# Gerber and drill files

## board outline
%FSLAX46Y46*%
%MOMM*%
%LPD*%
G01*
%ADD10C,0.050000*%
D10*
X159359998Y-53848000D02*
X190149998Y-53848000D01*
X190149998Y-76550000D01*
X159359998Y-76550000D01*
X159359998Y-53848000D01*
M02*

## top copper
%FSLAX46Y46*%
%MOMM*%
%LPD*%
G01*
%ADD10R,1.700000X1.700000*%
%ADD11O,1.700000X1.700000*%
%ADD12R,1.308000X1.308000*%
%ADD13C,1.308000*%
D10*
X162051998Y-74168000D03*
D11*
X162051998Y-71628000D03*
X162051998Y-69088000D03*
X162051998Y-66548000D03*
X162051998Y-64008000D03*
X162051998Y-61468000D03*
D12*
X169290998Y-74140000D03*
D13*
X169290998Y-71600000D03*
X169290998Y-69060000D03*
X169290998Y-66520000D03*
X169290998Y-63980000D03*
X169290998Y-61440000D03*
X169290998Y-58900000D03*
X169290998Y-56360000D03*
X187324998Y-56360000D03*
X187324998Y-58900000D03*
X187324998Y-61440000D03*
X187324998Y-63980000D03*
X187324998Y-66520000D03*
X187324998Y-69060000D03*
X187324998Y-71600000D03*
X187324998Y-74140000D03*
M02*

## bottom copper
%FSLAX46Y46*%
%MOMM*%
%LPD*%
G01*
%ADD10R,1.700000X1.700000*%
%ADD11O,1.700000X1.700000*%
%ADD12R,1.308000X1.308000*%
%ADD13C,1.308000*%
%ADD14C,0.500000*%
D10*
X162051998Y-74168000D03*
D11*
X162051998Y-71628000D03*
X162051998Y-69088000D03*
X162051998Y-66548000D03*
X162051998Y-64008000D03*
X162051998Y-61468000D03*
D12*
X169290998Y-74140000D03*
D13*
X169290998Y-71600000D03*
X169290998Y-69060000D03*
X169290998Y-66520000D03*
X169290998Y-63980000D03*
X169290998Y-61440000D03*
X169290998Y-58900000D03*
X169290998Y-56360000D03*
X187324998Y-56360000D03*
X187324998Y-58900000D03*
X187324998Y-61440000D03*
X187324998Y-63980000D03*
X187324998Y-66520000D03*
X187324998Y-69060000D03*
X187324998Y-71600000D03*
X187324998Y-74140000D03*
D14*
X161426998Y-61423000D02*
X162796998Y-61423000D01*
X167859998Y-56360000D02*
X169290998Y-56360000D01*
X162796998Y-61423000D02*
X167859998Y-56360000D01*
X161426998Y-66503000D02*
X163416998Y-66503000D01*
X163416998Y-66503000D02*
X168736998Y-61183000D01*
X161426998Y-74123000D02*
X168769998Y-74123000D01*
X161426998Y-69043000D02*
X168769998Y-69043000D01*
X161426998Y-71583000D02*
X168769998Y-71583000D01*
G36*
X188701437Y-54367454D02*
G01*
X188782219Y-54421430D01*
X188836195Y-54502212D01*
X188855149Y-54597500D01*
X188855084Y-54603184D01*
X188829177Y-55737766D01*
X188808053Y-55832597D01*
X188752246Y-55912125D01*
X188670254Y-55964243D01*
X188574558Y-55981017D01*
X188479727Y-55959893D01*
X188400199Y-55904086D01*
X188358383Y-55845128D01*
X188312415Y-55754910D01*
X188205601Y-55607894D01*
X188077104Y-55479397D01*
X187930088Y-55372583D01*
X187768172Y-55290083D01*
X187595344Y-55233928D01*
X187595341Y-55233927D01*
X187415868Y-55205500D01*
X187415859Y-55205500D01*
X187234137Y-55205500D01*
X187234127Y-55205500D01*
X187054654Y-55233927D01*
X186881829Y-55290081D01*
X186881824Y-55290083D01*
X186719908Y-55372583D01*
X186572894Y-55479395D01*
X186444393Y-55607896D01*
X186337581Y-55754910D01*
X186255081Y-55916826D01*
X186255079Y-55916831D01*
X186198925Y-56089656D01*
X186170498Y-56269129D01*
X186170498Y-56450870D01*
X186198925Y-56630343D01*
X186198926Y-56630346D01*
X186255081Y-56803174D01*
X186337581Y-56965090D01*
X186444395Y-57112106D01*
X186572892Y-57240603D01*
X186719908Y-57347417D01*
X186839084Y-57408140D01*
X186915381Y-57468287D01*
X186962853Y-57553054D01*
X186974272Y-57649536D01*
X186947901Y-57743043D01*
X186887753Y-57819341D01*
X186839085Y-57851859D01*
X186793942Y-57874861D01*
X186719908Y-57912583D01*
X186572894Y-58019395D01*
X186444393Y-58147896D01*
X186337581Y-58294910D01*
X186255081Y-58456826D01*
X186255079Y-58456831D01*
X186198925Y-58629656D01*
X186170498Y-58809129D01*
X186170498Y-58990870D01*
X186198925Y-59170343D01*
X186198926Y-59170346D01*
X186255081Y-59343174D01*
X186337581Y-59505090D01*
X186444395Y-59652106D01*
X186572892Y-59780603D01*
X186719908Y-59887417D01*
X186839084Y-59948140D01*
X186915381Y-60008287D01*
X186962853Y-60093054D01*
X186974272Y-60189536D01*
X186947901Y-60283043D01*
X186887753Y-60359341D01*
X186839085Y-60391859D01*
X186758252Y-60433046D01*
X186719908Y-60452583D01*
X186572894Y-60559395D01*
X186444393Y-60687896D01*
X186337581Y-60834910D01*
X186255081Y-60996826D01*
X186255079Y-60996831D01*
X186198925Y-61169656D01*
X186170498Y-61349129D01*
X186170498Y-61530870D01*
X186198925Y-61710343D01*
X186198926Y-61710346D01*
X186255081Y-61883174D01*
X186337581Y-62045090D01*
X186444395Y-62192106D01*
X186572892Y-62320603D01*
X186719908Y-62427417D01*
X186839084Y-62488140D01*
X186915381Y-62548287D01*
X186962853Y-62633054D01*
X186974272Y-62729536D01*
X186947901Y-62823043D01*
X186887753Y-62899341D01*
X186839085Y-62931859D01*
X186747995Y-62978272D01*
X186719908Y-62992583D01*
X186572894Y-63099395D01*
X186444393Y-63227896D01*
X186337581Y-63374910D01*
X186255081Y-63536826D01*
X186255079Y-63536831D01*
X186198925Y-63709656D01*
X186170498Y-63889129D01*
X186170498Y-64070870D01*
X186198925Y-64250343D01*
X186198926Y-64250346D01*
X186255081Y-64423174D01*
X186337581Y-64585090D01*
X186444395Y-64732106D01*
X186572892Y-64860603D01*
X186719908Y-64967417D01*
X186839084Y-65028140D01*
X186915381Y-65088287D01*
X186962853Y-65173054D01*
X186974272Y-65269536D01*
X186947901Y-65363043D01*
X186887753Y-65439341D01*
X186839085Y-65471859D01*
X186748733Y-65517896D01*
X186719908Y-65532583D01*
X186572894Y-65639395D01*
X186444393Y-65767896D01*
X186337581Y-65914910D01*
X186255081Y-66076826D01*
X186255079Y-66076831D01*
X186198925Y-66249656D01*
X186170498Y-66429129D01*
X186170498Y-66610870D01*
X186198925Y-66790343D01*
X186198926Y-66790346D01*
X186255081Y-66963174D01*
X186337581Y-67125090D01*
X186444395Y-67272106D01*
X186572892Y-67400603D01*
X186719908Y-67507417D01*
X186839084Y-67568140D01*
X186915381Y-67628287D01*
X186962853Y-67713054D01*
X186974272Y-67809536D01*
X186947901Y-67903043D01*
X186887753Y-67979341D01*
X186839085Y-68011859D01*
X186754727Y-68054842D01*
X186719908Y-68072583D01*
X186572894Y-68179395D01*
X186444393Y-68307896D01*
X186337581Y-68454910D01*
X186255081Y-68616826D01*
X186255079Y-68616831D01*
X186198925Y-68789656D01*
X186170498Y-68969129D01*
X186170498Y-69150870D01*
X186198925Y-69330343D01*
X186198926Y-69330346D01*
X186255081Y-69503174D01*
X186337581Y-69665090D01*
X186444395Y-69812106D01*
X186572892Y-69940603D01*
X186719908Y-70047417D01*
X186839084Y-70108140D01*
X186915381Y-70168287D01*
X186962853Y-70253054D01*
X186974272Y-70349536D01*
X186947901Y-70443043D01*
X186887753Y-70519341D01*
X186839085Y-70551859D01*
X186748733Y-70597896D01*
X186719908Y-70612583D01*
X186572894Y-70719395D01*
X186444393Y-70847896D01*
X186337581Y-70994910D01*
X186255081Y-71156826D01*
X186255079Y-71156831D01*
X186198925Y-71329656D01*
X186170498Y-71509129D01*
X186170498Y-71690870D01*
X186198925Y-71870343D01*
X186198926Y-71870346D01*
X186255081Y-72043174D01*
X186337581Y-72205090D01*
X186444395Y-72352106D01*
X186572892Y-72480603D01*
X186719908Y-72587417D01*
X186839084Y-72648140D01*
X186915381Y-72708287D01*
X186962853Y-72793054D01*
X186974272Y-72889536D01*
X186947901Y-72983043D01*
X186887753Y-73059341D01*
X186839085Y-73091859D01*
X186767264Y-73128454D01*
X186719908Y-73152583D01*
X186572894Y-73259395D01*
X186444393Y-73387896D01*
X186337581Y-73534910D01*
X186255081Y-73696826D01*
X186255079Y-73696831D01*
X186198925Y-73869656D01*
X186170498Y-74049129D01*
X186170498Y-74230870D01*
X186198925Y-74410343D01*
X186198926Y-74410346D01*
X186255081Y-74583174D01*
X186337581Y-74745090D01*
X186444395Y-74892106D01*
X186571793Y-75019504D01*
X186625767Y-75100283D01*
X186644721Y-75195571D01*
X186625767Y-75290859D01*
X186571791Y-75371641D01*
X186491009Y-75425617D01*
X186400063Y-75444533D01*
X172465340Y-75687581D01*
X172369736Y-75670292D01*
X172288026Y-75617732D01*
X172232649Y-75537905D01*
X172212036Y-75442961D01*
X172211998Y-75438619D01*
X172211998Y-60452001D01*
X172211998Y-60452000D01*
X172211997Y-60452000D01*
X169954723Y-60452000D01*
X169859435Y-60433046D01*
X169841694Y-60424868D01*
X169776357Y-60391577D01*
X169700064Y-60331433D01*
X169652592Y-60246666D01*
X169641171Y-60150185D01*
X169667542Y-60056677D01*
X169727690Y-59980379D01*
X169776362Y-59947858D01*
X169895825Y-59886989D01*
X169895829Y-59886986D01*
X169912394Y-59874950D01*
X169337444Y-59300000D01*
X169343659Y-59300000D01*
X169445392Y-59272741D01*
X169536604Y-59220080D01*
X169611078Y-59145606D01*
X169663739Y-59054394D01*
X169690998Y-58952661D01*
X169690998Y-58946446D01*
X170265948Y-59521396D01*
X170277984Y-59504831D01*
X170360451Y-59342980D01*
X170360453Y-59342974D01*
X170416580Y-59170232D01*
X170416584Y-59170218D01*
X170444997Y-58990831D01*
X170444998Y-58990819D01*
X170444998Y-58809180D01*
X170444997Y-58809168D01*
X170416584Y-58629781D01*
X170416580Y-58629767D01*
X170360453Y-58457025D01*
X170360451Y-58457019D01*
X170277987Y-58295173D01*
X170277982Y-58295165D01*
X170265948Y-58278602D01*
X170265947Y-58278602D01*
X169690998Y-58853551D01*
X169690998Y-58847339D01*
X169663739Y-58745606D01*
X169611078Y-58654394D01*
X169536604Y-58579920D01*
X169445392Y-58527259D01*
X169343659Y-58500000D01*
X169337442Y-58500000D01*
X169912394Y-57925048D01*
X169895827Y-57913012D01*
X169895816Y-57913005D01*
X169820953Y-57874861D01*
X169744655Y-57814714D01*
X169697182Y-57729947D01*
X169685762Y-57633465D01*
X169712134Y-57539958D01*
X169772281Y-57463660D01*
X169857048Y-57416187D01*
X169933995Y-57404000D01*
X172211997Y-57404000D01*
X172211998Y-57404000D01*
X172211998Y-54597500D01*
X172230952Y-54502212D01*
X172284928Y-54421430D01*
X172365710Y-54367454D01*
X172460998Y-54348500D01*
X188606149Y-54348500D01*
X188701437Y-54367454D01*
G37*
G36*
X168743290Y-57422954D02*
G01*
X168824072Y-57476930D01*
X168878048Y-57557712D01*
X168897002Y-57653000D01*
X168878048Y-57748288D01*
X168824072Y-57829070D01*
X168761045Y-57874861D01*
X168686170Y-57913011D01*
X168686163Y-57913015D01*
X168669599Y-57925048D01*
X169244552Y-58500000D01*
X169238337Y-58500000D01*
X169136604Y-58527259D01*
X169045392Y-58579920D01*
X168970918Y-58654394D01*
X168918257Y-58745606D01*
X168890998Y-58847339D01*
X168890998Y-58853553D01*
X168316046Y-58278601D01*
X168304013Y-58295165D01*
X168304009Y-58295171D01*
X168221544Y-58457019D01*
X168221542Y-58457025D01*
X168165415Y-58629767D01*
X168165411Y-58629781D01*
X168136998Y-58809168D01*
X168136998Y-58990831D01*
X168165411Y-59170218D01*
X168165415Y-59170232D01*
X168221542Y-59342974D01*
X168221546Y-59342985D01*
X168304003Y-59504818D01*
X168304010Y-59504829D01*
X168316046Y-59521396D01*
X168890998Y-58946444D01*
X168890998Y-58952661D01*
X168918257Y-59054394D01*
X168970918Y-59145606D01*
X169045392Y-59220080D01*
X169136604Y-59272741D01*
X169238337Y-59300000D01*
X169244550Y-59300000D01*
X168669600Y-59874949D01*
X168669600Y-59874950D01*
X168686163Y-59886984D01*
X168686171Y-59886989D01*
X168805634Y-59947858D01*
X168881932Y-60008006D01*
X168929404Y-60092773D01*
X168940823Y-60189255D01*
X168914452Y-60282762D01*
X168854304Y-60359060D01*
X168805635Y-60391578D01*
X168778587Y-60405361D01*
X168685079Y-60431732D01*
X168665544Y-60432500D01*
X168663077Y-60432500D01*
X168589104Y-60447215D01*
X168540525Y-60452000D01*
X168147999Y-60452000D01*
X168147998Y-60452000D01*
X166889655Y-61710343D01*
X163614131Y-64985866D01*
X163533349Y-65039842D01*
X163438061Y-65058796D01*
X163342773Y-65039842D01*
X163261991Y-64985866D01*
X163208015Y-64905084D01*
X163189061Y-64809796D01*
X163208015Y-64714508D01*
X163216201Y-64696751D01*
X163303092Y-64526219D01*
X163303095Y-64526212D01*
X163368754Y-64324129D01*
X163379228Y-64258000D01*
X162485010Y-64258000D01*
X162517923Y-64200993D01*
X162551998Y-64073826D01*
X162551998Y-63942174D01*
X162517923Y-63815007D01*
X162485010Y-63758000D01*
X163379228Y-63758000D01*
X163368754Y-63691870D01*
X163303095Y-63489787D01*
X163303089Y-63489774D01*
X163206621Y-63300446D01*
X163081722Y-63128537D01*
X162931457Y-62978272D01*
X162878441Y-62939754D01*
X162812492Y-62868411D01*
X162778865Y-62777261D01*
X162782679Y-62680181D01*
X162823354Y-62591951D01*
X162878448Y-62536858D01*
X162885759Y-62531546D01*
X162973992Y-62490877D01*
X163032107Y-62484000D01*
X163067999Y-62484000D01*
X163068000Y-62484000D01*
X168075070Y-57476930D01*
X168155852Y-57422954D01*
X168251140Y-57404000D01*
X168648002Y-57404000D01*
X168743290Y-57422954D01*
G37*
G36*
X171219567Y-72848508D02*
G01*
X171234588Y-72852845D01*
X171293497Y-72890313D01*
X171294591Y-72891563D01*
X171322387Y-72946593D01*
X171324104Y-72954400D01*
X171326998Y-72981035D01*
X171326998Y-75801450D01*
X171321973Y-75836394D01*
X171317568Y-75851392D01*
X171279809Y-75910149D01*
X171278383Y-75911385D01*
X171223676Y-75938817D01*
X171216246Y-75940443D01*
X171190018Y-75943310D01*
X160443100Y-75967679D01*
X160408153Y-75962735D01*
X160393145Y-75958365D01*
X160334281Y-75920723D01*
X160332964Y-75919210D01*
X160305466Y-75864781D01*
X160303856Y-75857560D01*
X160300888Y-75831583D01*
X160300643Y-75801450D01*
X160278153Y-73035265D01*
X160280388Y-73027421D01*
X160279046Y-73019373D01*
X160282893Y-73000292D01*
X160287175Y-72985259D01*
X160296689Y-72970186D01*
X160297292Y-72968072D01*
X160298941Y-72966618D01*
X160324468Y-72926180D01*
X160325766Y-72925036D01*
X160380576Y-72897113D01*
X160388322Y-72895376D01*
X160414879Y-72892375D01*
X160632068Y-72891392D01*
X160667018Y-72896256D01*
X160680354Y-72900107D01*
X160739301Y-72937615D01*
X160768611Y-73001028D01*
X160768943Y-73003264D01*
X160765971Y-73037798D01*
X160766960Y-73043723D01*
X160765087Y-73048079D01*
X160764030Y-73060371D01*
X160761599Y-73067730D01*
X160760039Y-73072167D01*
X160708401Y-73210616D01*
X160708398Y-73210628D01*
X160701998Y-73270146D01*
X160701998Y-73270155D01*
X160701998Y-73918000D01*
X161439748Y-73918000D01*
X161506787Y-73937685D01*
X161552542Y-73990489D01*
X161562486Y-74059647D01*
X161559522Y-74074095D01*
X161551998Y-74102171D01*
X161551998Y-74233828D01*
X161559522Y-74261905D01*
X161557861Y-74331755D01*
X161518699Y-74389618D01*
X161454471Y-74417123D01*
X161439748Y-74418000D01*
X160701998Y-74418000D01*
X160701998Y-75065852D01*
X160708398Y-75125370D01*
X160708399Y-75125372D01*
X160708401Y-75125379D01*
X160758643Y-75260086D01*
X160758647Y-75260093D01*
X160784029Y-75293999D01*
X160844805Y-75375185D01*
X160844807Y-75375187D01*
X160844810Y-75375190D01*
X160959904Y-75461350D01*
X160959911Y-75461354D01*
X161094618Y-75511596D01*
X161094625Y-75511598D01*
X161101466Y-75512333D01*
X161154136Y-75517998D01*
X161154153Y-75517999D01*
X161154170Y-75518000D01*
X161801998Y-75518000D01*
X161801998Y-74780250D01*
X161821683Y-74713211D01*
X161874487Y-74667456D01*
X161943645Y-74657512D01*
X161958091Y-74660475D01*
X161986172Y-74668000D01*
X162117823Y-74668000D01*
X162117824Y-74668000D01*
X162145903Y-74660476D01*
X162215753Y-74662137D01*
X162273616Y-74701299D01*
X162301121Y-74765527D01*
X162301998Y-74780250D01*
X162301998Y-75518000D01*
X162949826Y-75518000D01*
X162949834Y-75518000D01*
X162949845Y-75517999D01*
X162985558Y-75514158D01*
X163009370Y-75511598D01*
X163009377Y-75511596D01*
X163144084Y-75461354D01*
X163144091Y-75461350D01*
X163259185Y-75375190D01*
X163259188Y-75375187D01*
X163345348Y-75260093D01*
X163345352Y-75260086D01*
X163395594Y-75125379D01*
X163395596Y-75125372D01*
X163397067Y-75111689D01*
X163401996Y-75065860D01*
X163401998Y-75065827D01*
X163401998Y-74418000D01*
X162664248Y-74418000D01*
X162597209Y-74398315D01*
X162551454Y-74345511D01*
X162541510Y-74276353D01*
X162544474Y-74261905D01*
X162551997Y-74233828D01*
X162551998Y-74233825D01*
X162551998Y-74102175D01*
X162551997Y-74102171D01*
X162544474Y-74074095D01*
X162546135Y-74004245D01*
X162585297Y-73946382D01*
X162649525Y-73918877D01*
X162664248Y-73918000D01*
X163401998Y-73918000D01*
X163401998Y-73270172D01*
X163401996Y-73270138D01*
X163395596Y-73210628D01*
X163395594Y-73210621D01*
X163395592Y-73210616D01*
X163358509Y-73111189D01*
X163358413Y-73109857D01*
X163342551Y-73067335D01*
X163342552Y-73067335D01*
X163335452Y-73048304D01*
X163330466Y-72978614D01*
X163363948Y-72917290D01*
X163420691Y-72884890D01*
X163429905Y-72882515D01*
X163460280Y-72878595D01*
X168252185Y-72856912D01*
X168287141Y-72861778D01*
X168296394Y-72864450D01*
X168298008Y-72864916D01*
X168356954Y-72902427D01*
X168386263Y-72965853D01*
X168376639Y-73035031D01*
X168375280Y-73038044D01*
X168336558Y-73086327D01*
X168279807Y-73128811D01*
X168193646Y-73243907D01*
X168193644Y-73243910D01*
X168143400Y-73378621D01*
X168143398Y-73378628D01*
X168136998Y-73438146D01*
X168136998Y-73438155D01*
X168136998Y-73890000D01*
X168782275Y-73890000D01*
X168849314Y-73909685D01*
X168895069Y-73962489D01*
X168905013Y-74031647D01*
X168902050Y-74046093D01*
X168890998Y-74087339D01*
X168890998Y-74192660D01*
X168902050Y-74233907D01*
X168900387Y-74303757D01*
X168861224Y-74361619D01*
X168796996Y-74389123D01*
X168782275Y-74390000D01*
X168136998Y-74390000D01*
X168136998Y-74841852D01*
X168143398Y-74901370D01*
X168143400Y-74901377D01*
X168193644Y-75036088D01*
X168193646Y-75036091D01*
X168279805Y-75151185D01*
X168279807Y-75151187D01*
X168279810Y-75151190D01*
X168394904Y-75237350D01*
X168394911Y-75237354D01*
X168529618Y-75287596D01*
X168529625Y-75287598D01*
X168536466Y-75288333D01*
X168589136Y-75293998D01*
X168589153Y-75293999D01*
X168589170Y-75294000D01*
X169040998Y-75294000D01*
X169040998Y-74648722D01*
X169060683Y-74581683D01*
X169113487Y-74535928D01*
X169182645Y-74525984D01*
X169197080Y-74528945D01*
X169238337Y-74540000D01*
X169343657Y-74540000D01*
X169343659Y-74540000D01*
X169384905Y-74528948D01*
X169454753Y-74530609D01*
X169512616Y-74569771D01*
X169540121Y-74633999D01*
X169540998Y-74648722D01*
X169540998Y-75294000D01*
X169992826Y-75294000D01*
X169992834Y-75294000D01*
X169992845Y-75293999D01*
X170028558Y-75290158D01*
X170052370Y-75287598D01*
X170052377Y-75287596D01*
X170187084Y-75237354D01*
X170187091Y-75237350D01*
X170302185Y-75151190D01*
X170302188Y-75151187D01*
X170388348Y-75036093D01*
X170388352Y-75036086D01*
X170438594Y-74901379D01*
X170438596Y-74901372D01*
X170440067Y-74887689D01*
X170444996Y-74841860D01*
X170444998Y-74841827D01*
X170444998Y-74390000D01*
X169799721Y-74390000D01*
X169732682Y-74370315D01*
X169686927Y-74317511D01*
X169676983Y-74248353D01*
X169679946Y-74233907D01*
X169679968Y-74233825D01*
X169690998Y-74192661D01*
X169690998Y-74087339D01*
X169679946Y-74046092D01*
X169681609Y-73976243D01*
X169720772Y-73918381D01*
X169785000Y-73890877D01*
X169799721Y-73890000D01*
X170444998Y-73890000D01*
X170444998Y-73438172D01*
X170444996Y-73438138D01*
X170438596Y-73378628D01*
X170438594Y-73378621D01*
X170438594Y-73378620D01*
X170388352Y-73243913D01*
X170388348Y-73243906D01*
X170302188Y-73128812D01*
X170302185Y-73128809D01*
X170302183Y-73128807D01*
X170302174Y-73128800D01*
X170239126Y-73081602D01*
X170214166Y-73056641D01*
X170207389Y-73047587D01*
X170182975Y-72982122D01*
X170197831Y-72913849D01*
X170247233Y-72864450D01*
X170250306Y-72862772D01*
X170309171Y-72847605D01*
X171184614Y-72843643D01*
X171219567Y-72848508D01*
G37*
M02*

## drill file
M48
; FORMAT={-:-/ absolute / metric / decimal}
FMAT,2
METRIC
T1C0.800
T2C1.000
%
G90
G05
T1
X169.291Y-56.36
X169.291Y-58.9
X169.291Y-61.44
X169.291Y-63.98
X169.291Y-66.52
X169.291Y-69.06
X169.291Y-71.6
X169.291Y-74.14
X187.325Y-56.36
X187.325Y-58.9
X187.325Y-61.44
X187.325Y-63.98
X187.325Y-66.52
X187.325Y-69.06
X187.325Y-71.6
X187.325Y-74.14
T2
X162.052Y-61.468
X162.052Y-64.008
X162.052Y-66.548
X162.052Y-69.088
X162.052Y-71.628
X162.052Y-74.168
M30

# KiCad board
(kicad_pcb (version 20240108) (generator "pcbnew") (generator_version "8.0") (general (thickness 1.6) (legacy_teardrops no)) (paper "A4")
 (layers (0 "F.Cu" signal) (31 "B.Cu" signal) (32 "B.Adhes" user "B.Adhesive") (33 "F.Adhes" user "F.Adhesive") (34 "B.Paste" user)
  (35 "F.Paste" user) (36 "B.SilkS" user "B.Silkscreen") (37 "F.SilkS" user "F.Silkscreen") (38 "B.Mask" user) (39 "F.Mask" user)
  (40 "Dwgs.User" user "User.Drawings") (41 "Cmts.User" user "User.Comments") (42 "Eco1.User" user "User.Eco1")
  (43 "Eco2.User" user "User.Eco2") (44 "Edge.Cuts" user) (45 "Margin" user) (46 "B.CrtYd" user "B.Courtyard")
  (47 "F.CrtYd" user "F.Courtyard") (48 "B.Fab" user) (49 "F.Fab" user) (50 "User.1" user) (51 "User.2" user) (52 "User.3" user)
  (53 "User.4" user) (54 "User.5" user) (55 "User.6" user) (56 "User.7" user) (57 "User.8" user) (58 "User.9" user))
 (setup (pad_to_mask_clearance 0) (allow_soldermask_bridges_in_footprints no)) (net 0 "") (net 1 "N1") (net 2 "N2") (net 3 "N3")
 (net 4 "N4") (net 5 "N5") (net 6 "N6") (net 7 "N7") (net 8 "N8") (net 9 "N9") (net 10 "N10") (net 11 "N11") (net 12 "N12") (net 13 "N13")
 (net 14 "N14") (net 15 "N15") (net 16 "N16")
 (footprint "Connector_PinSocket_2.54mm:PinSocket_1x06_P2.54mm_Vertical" (layer "F.Cu") (at 162.051998 74.168 180)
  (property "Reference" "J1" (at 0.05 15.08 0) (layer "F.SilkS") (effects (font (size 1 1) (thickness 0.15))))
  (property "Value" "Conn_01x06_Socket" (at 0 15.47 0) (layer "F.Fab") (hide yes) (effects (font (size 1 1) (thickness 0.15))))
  (pad "1" thru_hole rect (at 0 0 180) (size 1.7 1.7) (drill 1) (layers "*.Cu" "*.Mask") (remove_unused_layers no) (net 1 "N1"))
  (pad "2" thru_hole oval (at 0 2.54 180) (size 1.7 1.7) (drill 1) (layers "*.Cu" "*.Mask") (remove_unused_layers no) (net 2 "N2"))
  (pad "3" thru_hole oval (at 0 5.08 180) (size 1.7 1.7) (drill 1) (layers "*.Cu" "*.Mask") (remove_unused_layers no) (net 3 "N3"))
  (pad "4" thru_hole oval (at 0 7.62 180) (size 1.7 1.7) (drill 1) (layers "*.Cu" "*.Mask") (remove_unused_layers no) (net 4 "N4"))
  (pad "5" thru_hole oval (at 0 10.16 180) (size 1.7 1.7) (drill 1) (layers "*.Cu" "*.Mask") (remove_unused_layers no) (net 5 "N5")
   (teardrops (best_length_ratio 0.5) (max_length 1) (best_width_ratio 1) (max_width 2) (curve_points 0) (filter_ratio 0.9) (enabled yes)
    (allow_two_segments yes) (prefer_zone_connections yes)))
  (pad "6" thru_hole oval (at 0 12.7 180) (size 1.7 1.7) (drill 1) (layers "*.Cu" "*.Mask") (remove_unused_layers no) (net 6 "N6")))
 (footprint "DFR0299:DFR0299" (layer "F.Cu") (at 178.307998 65.25 180)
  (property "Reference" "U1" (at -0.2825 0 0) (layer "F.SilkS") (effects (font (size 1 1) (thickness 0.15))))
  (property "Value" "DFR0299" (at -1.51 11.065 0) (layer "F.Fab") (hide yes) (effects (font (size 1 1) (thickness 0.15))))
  (pad "1" thru_hole rect (at 9.017 -8.89 180) (size 1.308 1.308) (drill 0.8) (layers "*.Cu" "*.Mask") (remove_unused_layers no)
   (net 1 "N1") (solder_mask_margin 0.102))
  (pad "2" thru_hole circle (at 9.017 -6.35 180) (size 1.308 1.308) (drill 0.8) (layers "*.Cu" "*.Mask") (remove_unused_layers no)
   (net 2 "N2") (solder_mask_margin 0.102))
  (pad "3" thru_hole circle (at 9.017 -3.81 180) (size 1.308 1.308) (drill 0.8) (layers "*.Cu" "*.Mask") (remove_unused_layers no)
   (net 3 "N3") (solder_mask_margin 0.102))
  (pad "4" thru_hole circle (at 9.017 -1.27 180) (size 1.308 1.308) (drill 0.8) (layers "*.Cu" "*.Mask") (remove_unused_layers no)
   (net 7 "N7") (solder_mask_margin 0.102))
  (pad "5" thru_hole circle (at 9.017 1.27 180) (size 1.308 1.308) (drill 0.8) (layers "*.Cu" "*.Mask") (remove_unused_layers no)
   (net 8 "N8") (solder_mask_margin 0.102))
  (pad "6" thru_hole circle (at 9.017 3.81 180) (size 1.308 1.308) (drill 0.8) (layers "*.Cu" "*.Mask") (remove_unused_layers no)
   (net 4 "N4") (solder_mask_margin 0.102))
  (pad "7" thru_hole circle (at 9.017 6.35 180) (size 1.308 1.308) (drill 0.8) (layers "*.Cu" "*.Mask") (remove_unused_layers no)
   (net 5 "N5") (solder_mask_margin 0.102))
  (pad "8" thru_hole circle (at 9.017 8.89 180) (size 1.308 1.308) (drill 0.8) (layers "*.Cu" "*.Mask") (remove_unused_layers no)
   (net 6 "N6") (solder_mask_margin 0.102))
  (pad "9" thru_hole circle (at -9.017 8.89 180) (size 1.308 1.308) (drill 0.8) (layers "*.Cu" "*.Mask") (remove_unused_layers no)
   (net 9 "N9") (solder_mask_margin 0.102))
  (pad "10" thru_hole circle (at -9.017 6.35 180) (size 1.308 1.308) (drill 0.8) (layers "*.Cu" "*.Mask") (remove_unused_layers no)
   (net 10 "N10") (solder_mask_margin 0.102))
  (pad "11" thru_hole circle (at -9.017 3.81 180) (size 1.308 1.308) (drill 0.8) (layers "*.Cu" "*.Mask") (remove_unused_layers no)
   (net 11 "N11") (solder_mask_margin 0.102))
  (pad "12" thru_hole circle (at -9.017 1.27 180) (size 1.308 1.308) (drill 0.8) (layers "*.Cu" "*.Mask") (remove_unused_layers no)
   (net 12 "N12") (solder_mask_margin 0.102))
  (pad "13" thru_hole circle (at -9.017 -1.27 180) (size 1.308 1.308) (drill 0.8) (layers "*.Cu" "*.Mask") (remove_unused_layers no)
   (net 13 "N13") (solder_mask_margin 0.102))
  (pad "14" thru_hole circle (at -9.017 -3.81 180) (size 1.308 1.308) (drill 0.8) (layers "*.Cu" "*.Mask") (remove_unused_layers no)
   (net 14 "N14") (solder_mask_margin 0.102))
  (pad "15" thru_hole circle (at -9.017 -6.35 180) (size 1.308 1.308) (drill 0.8) (layers "*.Cu" "*.Mask") (remove_unused_layers no)
   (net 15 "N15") (solder_mask_margin 0.102))
  (pad "16" thru_hole circle (at -9.017 -8.89 180) (size 1.308 1.308) (drill 0.8) (layers "*.Cu" "*.Mask") (remove_unused_layers no)
   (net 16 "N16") (solder_mask_margin 0.102)))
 (gr_rect (start 159.359998 53.848) (end 190.149998 76.55) (stroke (width 0.05) (type default)) (fill none) (layer "Edge.Cuts"))
 (segment (start 161.426998 61.423) (end 162.796998 61.423) (width 0.5) (layer "B.Cu") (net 6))
 (segment (start 167.859998 56.36) (end 169.290998 56.36) (width 0.5) (layer "B.Cu") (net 6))
 (segment (start 162.796998 61.423) (end 167.859998 56.36) (width 0.5) (layer "B.Cu") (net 6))
 (segment (start 161.426998 66.503) (end 163.416998 66.503) (width 0.5) (layer "B.Cu") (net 4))
 (segment (start 163.416998 66.503) (end 168.736998 61.183) (width 0.5) (layer "B.Cu") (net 4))
 (segment (start 161.426998 74.123) (end 168.769998 74.123) (width 0.5) (layer "B.Cu") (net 1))
 (segment (start 161.426998 69.043) (end 168.769998 69.043) (width 0.5) (layer "B.Cu") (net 3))
 (segment (start 161.426998 71.583) (end 168.769998 71.583) (width 0.5) (layer "B.Cu") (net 2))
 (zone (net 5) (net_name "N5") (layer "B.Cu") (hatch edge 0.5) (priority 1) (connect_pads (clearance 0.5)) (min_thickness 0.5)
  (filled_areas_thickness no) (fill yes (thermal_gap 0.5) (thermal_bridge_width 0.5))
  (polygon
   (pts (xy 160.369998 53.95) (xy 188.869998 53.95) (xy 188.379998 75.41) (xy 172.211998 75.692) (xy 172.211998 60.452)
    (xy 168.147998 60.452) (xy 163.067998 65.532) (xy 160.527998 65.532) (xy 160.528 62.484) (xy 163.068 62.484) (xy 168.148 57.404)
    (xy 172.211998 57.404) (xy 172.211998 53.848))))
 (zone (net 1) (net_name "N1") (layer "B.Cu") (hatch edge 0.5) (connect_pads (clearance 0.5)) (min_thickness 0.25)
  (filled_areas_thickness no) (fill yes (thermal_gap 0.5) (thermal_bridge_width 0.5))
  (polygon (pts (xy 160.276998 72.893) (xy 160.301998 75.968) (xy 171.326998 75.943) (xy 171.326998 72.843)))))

